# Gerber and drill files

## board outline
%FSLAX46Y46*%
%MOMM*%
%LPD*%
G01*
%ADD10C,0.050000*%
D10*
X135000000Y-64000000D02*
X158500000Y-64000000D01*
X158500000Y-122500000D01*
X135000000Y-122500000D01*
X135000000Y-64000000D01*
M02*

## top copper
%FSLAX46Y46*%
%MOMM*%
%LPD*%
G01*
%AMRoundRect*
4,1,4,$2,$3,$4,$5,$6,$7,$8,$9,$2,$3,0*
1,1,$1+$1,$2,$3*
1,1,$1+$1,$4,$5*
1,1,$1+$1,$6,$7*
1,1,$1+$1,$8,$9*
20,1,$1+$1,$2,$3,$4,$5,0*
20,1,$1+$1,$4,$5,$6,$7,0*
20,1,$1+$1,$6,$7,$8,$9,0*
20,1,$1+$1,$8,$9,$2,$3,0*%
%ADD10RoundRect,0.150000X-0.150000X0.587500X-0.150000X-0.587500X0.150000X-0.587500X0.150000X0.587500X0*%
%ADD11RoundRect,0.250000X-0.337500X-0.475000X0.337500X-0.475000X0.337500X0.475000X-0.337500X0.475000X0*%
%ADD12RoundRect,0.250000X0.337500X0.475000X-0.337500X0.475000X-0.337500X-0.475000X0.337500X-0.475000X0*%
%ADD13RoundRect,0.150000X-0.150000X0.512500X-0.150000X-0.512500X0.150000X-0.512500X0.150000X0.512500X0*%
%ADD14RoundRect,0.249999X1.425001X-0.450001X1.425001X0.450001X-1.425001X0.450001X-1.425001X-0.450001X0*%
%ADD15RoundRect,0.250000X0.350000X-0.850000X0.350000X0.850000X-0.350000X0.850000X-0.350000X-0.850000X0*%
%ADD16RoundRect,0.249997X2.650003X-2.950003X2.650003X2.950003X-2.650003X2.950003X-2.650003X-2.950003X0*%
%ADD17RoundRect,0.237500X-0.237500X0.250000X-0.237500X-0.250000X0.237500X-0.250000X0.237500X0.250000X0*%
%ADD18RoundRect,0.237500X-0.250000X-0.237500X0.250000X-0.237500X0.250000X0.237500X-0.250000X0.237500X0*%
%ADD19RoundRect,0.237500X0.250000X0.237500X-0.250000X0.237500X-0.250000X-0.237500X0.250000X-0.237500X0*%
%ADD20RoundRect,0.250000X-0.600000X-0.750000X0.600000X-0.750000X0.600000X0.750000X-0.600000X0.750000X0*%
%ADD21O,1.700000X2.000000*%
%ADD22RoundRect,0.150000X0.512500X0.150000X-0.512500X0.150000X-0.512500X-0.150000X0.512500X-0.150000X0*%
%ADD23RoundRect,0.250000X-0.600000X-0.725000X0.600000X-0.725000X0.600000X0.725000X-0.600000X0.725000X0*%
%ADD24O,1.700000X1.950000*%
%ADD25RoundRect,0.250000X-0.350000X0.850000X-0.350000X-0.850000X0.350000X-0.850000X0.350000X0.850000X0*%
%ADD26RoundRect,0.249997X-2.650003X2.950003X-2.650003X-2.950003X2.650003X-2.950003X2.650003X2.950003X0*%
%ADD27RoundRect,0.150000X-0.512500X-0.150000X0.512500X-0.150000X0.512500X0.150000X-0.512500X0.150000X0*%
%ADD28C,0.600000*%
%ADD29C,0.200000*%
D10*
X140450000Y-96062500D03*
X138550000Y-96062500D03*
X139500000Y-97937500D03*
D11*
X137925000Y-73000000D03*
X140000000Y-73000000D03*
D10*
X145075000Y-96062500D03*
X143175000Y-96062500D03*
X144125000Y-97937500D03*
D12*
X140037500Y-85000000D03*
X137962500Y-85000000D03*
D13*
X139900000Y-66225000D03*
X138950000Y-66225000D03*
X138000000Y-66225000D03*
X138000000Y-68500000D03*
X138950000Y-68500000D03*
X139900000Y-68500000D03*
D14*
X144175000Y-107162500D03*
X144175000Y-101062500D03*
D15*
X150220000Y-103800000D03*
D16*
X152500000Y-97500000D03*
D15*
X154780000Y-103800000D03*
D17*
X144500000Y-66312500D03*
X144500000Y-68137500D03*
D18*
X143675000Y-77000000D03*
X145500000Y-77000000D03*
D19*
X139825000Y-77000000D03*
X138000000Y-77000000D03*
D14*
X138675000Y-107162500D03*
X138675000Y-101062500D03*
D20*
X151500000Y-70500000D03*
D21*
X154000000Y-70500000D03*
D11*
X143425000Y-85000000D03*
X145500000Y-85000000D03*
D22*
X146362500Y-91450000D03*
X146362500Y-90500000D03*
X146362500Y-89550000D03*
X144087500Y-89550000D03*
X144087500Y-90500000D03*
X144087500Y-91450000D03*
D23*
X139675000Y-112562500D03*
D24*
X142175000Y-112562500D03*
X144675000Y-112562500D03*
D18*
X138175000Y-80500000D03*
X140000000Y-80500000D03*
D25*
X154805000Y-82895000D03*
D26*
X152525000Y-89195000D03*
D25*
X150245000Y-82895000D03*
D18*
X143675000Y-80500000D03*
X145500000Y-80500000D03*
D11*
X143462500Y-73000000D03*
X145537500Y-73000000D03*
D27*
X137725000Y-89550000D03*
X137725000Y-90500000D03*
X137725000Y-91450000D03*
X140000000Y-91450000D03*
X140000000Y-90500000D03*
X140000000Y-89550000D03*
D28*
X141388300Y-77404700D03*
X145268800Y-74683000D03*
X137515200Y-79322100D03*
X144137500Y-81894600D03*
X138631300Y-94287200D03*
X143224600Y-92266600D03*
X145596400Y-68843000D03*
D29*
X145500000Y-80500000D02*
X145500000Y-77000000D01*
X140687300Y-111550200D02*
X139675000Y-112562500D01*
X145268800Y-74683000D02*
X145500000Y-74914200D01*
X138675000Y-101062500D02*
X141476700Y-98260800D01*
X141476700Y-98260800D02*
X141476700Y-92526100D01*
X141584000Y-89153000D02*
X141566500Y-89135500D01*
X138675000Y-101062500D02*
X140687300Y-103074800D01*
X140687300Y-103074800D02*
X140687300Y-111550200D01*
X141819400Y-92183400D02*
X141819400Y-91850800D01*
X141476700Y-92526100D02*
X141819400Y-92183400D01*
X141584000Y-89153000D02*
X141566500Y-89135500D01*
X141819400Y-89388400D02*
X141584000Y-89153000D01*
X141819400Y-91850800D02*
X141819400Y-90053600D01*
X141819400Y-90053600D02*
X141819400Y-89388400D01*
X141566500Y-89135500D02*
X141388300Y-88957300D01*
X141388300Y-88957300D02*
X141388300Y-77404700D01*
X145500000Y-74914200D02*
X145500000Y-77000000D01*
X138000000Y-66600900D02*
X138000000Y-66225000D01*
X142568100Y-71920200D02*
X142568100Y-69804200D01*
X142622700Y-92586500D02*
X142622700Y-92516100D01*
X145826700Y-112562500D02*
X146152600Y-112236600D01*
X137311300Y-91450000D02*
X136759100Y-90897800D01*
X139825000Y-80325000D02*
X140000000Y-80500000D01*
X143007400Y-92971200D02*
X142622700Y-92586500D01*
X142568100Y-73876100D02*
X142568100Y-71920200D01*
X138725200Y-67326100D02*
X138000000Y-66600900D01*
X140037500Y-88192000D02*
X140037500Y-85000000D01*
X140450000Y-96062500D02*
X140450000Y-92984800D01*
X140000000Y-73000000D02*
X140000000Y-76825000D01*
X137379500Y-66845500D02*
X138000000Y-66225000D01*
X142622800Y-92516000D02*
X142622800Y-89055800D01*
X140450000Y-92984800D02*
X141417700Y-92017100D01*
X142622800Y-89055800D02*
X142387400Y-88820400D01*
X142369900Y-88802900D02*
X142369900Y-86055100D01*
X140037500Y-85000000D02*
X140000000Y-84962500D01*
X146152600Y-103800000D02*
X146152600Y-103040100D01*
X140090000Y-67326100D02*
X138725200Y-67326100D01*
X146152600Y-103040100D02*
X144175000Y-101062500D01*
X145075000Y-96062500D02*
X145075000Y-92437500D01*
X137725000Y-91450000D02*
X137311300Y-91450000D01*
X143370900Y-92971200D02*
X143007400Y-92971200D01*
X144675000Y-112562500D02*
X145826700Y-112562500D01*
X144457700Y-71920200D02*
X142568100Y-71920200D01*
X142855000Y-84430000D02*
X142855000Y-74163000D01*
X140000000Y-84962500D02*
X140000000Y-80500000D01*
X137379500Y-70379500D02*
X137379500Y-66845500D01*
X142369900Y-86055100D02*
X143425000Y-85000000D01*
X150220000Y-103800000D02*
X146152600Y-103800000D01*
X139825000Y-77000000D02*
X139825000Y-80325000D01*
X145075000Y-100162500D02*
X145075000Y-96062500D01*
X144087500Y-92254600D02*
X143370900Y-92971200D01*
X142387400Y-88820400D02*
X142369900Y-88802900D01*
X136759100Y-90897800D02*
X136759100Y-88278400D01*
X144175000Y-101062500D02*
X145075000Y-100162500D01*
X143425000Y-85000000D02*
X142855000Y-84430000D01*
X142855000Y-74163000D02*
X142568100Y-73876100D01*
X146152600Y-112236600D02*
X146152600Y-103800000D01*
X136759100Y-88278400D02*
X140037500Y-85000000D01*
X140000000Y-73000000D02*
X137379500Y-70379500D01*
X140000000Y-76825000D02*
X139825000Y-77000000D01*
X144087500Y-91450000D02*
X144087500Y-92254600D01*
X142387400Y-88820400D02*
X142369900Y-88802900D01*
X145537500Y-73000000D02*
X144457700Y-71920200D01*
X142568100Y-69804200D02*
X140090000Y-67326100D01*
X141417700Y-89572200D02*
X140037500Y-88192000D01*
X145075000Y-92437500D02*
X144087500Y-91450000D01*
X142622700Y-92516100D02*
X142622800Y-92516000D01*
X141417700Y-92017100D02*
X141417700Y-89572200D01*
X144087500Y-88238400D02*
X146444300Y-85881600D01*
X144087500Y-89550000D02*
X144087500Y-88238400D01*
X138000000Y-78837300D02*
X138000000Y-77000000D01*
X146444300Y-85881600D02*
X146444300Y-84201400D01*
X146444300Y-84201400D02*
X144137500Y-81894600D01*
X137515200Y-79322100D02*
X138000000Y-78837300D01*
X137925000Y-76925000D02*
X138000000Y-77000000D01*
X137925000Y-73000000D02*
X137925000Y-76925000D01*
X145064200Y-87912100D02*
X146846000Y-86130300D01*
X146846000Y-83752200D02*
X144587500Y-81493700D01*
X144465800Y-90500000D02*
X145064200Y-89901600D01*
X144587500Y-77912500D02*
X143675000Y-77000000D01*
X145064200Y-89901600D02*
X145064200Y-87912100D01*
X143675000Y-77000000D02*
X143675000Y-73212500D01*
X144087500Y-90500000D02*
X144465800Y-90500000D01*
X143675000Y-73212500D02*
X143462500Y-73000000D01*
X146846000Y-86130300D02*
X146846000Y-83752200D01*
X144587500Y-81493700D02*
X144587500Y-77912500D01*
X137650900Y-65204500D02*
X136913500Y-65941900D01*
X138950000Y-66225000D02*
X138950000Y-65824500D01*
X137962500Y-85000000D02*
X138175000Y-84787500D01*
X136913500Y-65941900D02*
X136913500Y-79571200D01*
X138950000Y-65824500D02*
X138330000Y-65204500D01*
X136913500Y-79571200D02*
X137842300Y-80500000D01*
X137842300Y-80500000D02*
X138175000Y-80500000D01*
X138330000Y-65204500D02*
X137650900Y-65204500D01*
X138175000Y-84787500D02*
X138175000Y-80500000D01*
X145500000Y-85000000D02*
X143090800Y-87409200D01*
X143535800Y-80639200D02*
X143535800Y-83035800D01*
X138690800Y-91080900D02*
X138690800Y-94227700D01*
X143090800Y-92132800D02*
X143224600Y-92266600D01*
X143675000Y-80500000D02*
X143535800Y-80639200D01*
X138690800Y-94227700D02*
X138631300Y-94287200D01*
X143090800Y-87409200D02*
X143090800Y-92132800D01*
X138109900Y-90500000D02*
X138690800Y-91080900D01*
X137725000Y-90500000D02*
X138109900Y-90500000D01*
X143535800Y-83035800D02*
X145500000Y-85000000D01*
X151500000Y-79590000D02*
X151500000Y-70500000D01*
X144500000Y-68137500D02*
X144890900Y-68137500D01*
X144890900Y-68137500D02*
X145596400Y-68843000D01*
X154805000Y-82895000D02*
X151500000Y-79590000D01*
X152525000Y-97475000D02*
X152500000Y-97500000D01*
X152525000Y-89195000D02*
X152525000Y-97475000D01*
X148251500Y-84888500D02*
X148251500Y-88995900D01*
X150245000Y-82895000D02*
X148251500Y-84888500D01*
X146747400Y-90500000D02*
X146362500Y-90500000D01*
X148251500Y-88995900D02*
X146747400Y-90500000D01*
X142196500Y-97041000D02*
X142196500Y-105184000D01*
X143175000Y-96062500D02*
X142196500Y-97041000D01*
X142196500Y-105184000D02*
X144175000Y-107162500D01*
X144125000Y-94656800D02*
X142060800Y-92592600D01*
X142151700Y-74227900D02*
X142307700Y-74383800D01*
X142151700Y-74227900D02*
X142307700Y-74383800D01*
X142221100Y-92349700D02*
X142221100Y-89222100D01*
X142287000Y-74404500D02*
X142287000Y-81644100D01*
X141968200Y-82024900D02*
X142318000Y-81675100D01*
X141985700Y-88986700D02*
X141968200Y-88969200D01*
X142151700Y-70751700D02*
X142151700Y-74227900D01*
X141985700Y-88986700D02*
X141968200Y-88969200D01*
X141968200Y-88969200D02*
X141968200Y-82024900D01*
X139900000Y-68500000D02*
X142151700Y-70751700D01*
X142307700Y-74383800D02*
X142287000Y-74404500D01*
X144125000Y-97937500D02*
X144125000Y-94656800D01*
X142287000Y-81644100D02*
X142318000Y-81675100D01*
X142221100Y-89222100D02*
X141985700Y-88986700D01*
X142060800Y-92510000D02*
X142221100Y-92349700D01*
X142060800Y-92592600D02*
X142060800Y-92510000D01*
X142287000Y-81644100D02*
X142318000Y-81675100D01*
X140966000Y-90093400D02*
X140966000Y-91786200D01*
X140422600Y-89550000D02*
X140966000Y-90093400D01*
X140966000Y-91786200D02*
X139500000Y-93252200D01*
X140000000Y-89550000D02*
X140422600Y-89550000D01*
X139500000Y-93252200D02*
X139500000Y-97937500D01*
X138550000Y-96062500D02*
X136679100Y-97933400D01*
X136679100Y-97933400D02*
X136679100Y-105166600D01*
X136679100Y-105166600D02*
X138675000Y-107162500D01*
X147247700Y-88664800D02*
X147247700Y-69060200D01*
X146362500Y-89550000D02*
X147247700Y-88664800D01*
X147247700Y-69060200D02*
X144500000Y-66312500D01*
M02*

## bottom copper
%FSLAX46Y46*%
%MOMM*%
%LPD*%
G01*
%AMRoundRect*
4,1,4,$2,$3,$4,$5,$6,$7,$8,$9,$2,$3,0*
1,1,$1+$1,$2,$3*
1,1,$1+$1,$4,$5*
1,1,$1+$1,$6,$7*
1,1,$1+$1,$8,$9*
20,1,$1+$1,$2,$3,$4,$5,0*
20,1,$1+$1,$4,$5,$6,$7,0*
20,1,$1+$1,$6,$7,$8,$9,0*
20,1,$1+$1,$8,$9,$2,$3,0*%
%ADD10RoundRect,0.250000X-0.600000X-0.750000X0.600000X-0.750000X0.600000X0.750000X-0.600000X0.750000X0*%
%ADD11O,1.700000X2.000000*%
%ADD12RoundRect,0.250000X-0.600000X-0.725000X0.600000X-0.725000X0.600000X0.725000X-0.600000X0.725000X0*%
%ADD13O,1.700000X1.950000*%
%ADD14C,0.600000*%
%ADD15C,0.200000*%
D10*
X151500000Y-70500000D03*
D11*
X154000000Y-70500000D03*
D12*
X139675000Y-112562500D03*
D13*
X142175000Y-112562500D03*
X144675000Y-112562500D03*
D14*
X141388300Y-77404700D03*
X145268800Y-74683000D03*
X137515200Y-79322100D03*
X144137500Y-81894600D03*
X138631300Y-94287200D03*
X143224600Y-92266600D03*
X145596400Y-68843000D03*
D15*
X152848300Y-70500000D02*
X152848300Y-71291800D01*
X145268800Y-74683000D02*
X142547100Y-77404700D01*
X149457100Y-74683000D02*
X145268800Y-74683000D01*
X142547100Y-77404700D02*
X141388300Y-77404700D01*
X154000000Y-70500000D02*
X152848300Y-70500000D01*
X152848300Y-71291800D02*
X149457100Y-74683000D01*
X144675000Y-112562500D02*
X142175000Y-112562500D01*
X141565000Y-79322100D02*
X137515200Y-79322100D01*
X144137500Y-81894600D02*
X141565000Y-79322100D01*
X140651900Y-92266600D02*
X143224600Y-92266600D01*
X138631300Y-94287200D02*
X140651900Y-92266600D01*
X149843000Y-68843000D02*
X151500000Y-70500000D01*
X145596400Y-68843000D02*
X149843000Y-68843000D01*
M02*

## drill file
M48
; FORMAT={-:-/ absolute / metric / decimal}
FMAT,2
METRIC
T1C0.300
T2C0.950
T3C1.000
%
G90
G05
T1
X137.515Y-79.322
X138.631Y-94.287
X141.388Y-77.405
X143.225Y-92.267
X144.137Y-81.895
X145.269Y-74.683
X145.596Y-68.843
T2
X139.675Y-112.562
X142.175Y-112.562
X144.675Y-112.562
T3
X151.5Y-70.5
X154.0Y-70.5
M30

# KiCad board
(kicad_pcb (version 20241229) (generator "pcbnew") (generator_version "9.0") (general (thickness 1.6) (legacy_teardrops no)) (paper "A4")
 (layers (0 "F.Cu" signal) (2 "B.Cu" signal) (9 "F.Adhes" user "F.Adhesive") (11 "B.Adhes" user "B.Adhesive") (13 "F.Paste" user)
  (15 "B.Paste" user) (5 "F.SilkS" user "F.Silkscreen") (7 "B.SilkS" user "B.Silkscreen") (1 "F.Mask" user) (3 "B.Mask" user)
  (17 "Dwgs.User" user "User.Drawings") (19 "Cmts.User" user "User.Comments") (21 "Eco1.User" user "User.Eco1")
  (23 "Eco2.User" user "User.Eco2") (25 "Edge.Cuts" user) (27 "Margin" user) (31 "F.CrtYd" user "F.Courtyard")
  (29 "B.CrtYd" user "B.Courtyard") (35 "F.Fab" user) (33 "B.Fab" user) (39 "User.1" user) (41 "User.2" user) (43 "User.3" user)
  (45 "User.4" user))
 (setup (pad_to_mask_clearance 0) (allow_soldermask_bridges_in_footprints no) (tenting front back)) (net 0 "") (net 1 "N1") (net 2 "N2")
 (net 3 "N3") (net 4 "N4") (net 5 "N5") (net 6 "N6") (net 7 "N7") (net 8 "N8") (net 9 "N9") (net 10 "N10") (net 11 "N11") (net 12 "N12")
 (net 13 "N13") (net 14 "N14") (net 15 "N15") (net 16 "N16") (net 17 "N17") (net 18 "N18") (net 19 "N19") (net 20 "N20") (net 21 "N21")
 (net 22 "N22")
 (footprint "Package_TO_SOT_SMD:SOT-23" (layer "F.Cu") (at 139.5 97 -90)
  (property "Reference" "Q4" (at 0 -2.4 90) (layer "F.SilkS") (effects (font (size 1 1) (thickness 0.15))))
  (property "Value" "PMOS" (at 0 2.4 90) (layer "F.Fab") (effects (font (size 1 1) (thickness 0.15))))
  (pad "1" smd roundrect (at -0.9375 -0.95 270) (size 1.475 0.6) (layers "F.Cu" "F.Mask" "F.Paste") (roundrect_rratio 0.25) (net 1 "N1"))
  (pad "2" smd roundrect (at -0.9375 0.95 270) (size 1.475 0.6) (layers "F.Cu" "F.Mask" "F.Paste") (roundrect_rratio 0.25) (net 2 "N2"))
  (pad "3" smd roundrect (at 0.9375 0 270) (size 1.475 0.6) (layers "F.Cu" "F.Mask" "F.Paste") (roundrect_rratio 0.25) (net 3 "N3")))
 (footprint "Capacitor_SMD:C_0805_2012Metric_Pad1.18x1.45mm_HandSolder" (layer "F.Cu") (at 138.9625 73)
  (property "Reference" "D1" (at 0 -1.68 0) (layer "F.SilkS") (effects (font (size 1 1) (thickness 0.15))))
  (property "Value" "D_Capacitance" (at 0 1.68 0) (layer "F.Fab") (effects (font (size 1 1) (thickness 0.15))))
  (pad "1" smd roundrect (at -1.0375 0) (size 1.175 1.45) (layers "F.Cu" "F.Mask" "F.Paste") (roundrect_rratio 0.212766) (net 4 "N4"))
  (pad "2" smd roundrect (at 1.0375 0) (size 1.175 1.45) (layers "F.Cu" "F.Mask" "F.Paste") (roundrect_rratio 0.212766) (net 1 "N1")))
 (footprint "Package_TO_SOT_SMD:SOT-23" (layer "F.Cu") (at 144.125 97 -90)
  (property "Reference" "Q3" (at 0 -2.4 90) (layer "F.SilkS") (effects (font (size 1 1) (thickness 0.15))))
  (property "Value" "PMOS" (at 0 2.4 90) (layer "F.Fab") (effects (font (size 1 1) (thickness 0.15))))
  (pad "1" smd roundrect (at -0.9375 -0.95 270) (size 1.475 0.6) (layers "F.Cu" "F.Mask" "F.Paste") (roundrect_rratio 0.25) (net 1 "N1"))
  (pad "2" smd roundrect (at -0.9375 0.95 270) (size 1.475 0.6) (layers "F.Cu" "F.Mask" "F.Paste") (roundrect_rratio 0.25) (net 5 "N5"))
  (pad "3" smd roundrect (at 0.9375 0 270) (size 1.475 0.6) (layers "F.Cu" "F.Mask" "F.Paste") (roundrect_rratio 0.25) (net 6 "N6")))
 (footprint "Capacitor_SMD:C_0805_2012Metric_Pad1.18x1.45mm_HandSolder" (layer "F.Cu") (at 139 85 180)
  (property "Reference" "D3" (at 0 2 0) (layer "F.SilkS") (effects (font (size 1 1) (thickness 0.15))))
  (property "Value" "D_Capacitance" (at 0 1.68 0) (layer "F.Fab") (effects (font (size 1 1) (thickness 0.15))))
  (pad "1" smd roundrect (at -1.0375 0 180) (size 1.175 1.45) (layers "F.Cu" "F.Mask" "F.Paste") (roundrect_rratio 0.212766) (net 1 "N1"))
  (pad "2" smd roundrect (at 1.0375 0 180) (size 1.175 1.45) (layers "F.Cu" "F.Mask" "F.Paste") (roundrect_rratio 0.212766) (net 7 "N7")))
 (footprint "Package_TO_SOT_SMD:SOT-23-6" (layer "F.Cu") (at 138.95 67.3625 -90)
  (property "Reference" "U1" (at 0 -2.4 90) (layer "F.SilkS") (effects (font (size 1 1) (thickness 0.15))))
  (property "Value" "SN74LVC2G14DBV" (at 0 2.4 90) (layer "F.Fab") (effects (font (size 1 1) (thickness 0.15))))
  (pad "1" smd roundrect (at -1.1375 -0.95 270) (size 1.325 0.6) (layers "F.Cu" "F.Mask" "F.Paste") (roundrect_rratio 0.25) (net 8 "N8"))
  (pad "2" smd roundrect (at -1.1375 0 270) (size 1.325 0.6) (layers "F.Cu" "F.Mask" "F.Paste") (roundrect_rratio 0.25) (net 7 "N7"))
  (pad "3" smd roundrect (at -1.1375 0.95 270) (size 1.325 0.6) (layers "F.Cu" "F.Mask" "F.Paste") (roundrect_rratio 0.25) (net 1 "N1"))
  (pad "4" smd roundrect (at 1.1375 0.95 270) (size 1.325 0.6) (layers "F.Cu" "F.Mask" "F.Paste") (roundrect_rratio 0.25) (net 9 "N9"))
  (pad "5" smd roundrect (at 1.1375 0 270) (size 1.325 0.6) (layers "F.Cu" "F.Mask" "F.Paste") (roundrect_rratio 0.25) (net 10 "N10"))
  (pad "6" smd roundrect (at 1.1375 -0.95 270) (size 1.325 0.6) (layers "F.Cu" "F.Mask" "F.Paste") (roundrect_rratio 0.25) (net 6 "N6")))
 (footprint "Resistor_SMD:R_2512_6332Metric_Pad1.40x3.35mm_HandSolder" (layer "F.Cu") (at 144.175 104.1125 90)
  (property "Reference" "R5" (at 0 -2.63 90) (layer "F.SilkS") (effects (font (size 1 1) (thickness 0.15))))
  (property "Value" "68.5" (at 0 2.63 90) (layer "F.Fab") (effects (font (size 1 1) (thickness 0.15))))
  (pad "1" smd roundrect (at -3.05 0 90) (size 1.4 3.35) (layers "F.Cu" "F.Mask" "F.Paste") (roundrect_rratio 0.178571) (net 5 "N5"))
  (pad "2" smd roundrect (at 3.05 0 90) (size 1.4 3.35) (layers "F.Cu" "F.Mask" "F.Paste") (roundrect_rratio 0.178571) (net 1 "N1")))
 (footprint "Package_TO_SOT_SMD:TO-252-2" (layer "F.Cu") (at 152.5 98.76 90)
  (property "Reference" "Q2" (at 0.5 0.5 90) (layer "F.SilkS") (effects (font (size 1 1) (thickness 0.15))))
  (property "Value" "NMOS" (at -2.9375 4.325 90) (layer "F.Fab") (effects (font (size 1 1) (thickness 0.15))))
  (pad "" smd roundrect (at -0.415 -1.525 90) (size 3.05 2.75) (layers "F.Paste") (roundrect_rratio 0.090909))
  (pad "" smd roundrect (at -0.415 1.525 90) (size 3.05 2.75) (layers "F.Paste") (roundrect_rratio 0.090909))
  (pad "" smd roundrect (at 2.935 -1.525 90) (size 3.05 2.75) (layers "F.Paste") (roundrect_rratio 0.090909))
  (pad "" smd roundrect (at 2.935 1.525 90) (size 3.05 2.75) (layers "F.Paste") (roundrect_rratio 0.090909))
  (pad "1" smd roundrect (at -5.04 -2.28 90) (size 2.2 1.2) (layers "F.Cu" "F.Mask" "F.Paste") (roundrect_rratio 0.208333) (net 1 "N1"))
  (pad "2" smd roundrect (at 1.26 0 90) (size 6.4 5.8) (layers "F.Cu" "F.Mask") (roundrect_rratio 0.043103) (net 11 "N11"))
  (pad "3" smd roundrect (at -5.04 2.28 90) (size 2.2 1.2) (layers "F.Cu" "F.Mask" "F.Paste") (roundrect_rratio 0.208333) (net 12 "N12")))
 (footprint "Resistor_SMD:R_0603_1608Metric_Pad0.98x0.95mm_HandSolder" (layer "F.Cu") (at 144.5 67.225 -90)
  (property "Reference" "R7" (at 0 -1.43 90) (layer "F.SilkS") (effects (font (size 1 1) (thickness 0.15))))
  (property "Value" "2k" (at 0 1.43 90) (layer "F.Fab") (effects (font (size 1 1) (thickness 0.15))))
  (pad "1" smd roundrect (at -0.9125 0 270) (size 0.975 0.95) (layers "F.Cu" "F.Mask" "F.Paste") (roundrect_rratio 0.25) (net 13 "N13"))
  (pad "2" smd roundrect (at 0.9125 0 270) (size 0.975 0.95) (layers "F.Cu" "F.Mask" "F.Paste") (roundrect_rratio 0.25) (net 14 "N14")))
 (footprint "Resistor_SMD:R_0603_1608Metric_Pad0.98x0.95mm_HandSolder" (layer "F.Cu") (at 144.5875 77)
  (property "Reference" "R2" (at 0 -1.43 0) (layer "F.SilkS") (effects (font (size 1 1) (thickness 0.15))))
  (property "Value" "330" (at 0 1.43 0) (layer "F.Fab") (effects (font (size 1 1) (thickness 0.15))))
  (pad "1" smd roundrect (at -0.9125 0) (size 0.975 0.95) (layers "F.Cu" "F.Mask" "F.Paste") (roundrect_rratio 0.25) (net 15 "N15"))
  (pad "2" smd roundrect (at 0.9125 0) (size 0.975 0.95) (layers "F.Cu" "F.Mask" "F.Paste") (roundrect_rratio 0.25) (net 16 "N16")))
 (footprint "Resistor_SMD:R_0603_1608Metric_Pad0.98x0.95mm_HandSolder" (layer "F.Cu") (at 138.9125 77 180)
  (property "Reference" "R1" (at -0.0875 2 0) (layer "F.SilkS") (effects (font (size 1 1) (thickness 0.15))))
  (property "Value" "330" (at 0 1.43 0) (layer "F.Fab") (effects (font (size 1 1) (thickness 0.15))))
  (pad "1" smd roundrect (at -0.9125 0 180) (size 0.975 0.95) (layers "F.Cu" "F.Mask" "F.Paste") (roundrect_rratio 0.25) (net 1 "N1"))
  (pad "2" smd roundrect (at 0.9125 0 180) (size 0.975 0.95) (layers "F.Cu" "F.Mask" "F.Paste") (roundrect_rratio 0.25) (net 4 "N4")))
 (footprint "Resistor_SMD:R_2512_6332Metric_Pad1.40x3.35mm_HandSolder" (layer "F.Cu") (at 138.675 104.1125 90)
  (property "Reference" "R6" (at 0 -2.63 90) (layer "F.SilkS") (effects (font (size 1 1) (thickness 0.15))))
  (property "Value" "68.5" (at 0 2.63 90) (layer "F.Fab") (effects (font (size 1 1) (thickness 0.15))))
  (pad "1" smd roundrect (at -3.05 0 90) (size 1.4 3.35) (layers "F.Cu" "F.Mask" "F.Paste") (roundrect_rratio 0.178571) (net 2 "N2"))
  (pad "2" smd roundrect (at 3.05 0 90) (size 1.4 3.35) (layers "F.Cu" "F.Mask" "F.Paste") (roundrect_rratio 0.178571) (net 16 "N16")))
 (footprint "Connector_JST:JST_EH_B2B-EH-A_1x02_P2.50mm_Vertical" (layer "F.Cu") (at 151.5 70.5)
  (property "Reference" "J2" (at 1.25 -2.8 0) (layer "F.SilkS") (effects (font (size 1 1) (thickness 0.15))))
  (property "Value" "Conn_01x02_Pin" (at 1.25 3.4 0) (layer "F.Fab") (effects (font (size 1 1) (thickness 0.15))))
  (pad "1" thru_hole roundrect (at 0 0) (size 1.7 2) (drill 1) (layers "*.Cu" "*.Mask") (remove_unused_layers no)
   (roundrect_rratio 0.147059) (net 14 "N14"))
  (pad "2" thru_hole oval (at 2.5 0) (size 1.7 2) (drill 1) (layers "*.Cu" "*.Mask") (remove_unused_layers no) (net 16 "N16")))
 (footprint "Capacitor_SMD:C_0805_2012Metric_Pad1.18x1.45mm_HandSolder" (layer "F.Cu") (at 144.4625 85)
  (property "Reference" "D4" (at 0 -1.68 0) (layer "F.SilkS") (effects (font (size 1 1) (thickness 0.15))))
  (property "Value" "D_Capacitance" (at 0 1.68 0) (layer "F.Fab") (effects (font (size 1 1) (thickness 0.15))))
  (pad "1" smd roundrect (at -1.0375 0) (size 1.175 1.45) (layers "F.Cu" "F.Mask" "F.Paste") (roundrect_rratio 0.212766) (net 1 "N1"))
  (pad "2" smd roundrect (at 1.0375 0) (size 1.175 1.45) (layers "F.Cu" "F.Mask" "F.Paste") (roundrect_rratio 0.212766) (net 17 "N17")))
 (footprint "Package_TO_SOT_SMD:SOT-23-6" (layer "F.Cu") (at 145.225 90.5 180)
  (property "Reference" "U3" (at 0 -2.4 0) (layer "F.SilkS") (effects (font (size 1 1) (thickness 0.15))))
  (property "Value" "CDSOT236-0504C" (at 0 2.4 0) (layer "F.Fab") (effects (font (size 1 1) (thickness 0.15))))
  (pad "1" smd roundrect (at -1.1375 -0.95 180) (size 1.325 0.6) (layers "F.Cu" "F.Mask" "F.Paste") (roundrect_rratio 0.25) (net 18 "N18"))
  (pad "2" smd roundrect (at -1.1375 0 180) (size 1.325 0.6) (layers "F.Cu" "F.Mask" "F.Paste") (roundrect_rratio 0.25) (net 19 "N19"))
  (pad "3" smd roundrect (at -1.1375 0.95 180) (size 1.325 0.6) (layers "F.Cu" "F.Mask" "F.Paste") (roundrect_rratio 0.25) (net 13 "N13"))
  (pad "4" smd roundrect (at 1.1375 0.95 180) (size 1.325 0.6) (layers "F.Cu" "F.Mask" "F.Paste") (roundrect_rratio 0.25) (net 4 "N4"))
  (pad "5" smd roundrect (at 1.1375 0 180) (size 1.325 0.6) (layers "F.Cu" "F.Mask" "F.Paste") (roundrect_rratio 0.25) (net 15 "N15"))
  (pad "6" smd roundrect (at 1.1375 -0.95 180) (size 1.325 0.6) (layers "F.Cu" "F.Mask" "F.Paste") (roundrect_rratio 0.25) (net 1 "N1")))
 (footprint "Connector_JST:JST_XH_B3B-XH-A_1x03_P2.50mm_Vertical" (layer "F.Cu") (at 139.675 112.5625)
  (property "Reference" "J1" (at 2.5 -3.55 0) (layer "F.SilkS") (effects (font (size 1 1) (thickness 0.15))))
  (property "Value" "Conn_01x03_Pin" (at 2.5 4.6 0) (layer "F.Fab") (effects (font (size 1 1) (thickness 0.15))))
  (pad "1" thru_hole roundrect (at 0 0) (size 1.7 1.95) (drill 0.95) (layers "*.Cu" "*.Mask") (remove_unused_layers no)
   (roundrect_rratio 0.147059) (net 16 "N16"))
  (pad "2" thru_hole oval (at 2.5 0) (size 1.7 1.95) (drill 0.95) (layers "*.Cu" "*.Mask") (remove_unused_layers no) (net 1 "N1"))
  (pad "3" thru_hole oval (at 5 0) (size 1.7 1.95) (drill 0.95) (layers "*.Cu" "*.Mask") (remove_unused_layers no) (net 1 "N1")))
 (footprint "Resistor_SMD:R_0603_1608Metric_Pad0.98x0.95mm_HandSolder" (layer "F.Cu") (at 139.0875 80.5)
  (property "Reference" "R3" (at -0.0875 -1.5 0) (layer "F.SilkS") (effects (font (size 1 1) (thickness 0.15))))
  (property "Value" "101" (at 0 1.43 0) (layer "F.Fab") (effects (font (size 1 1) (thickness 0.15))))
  (pad "1" smd roundrect (at -0.9125 0) (size 0.975 0.95) (layers "F.Cu" "F.Mask" "F.Paste") (roundrect_rratio 0.25) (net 7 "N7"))
  (pad "2" smd roundrect (at 0.9125 0) (size 0.975 0.95) (layers "F.Cu" "F.Mask" "F.Paste") (roundrect_rratio 0.25) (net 1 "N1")))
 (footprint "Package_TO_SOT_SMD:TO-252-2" (layer "F.Cu") (at 152.525 87.935 -90)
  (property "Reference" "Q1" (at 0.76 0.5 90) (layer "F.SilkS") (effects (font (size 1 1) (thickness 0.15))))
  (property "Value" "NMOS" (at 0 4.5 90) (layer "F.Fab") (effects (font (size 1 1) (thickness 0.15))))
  (pad "" smd roundrect (at -0.415 -1.525 270) (size 3.05 2.75) (layers "F.Paste") (roundrect_rratio 0.090909))
  (pad "" smd roundrect (at -0.415 1.525 270) (size 3.05 2.75) (layers "F.Paste") (roundrect_rratio 0.090909))
  (pad "" smd roundrect (at 2.935 -1.525 270) (size 3.05 2.75) (layers "F.Paste") (roundrect_rratio 0.090909))
  (pad "" smd roundrect (at 2.935 1.525 270) (size 3.05 2.75) (layers "F.Paste") (roundrect_rratio 0.090909))
  (pad "1" smd roundrect (at -5.04 -2.28 270) (size 2.2 1.2) (layers "F.Cu" "F.Mask" "F.Paste") (roundrect_rratio 0.208333) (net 14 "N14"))
  (pad "2" smd roundrect (at 1.26 0 270) (size 6.4 5.8) (layers "F.Cu" "F.Mask") (roundrect_rratio 0.043103) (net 11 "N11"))
  (pad "3" smd roundrect (at -5.04 2.28 270) (size 2.2 1.2) (layers "F.Cu" "F.Mask" "F.Paste") (roundrect_rratio 0.208333) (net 19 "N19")))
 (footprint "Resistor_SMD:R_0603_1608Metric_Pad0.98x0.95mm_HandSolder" (layer "F.Cu") (at 144.5875 80.5)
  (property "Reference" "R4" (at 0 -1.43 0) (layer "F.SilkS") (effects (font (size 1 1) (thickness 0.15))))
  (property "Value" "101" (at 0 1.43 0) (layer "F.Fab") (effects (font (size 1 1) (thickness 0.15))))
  (pad "1" smd roundrect (at -0.9125 0) (size 0.975 0.95) (layers "F.Cu" "F.Mask" "F.Paste") (roundrect_rratio 0.25) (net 17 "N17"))
  (pad "2" smd roundrect (at 0.9125 0) (size 0.975 0.95) (layers "F.Cu" "F.Mask" "F.Paste") (roundrect_rratio 0.25) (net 16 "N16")))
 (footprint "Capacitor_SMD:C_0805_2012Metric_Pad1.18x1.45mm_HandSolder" (layer "F.Cu") (at 144.5 73)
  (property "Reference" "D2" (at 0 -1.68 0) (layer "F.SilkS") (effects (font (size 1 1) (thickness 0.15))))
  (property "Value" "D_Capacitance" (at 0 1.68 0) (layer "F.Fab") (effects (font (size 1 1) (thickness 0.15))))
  (pad "1" smd roundrect (at -1.0375 0) (size 1.175 1.45) (layers "F.Cu" "F.Mask" "F.Paste") (roundrect_rratio 0.212766) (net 15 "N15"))
  (pad "2" smd roundrect (at 1.0375 0) (size 1.175 1.45) (layers "F.Cu" "F.Mask" "F.Paste") (roundrect_rratio 0.212766) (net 1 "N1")))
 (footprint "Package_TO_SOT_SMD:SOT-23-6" (layer "F.Cu") (at 138.8625 90.5)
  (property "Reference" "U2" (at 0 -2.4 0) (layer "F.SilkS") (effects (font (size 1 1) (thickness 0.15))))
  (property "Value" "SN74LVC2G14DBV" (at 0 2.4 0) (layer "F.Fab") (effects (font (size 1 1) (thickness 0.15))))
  (pad "1" smd roundrect (at -1.1375 -0.95) (size 1.325 0.6) (layers "F.Cu" "F.Mask" "F.Paste") (roundrect_rratio 0.25) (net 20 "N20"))
  (pad "2" smd roundrect (at -1.1375 0) (size 1.325 0.6) (layers "F.Cu" "F.Mask" "F.Paste") (roundrect_rratio 0.25) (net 17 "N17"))
  (pad "3" smd roundrect (at -1.1375 0.95) (size 1.325 0.6) (layers "F.Cu" "F.Mask" "F.Paste") (roundrect_rratio 0.25) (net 1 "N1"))
  (pad "4" smd roundrect (at 1.1375 0.95) (size 1.325 0.6) (layers "F.Cu" "F.Mask" "F.Paste") (roundrect_rratio 0.25) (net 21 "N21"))
  (pad "5" smd roundrect (at 1.1375 0) (size 1.325 0.6) (layers "F.Cu" "F.Mask" "F.Paste") (roundrect_rratio 0.25) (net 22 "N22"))
  (pad "6" smd roundrect (at 1.1375 -0.95) (size 1.325 0.6) (layers "F.Cu" "F.Mask" "F.Paste") (roundrect_rratio 0.25) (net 3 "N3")))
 (gr_rect (start 135 64) (end 158.5 122.5) (stroke (width 0.05) (type default)) (fill no) (layer "Edge.Cuts"))
 (segment (start 145.5 80.5) (end 145.5 77) (width 0.2) (layer "F.Cu") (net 16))
 (segment (start 140.6873 111.5502) (end 139.675 112.5625) (width 0.2) (layer "F.Cu") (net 16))
 (segment (start 145.2688 74.683) (end 145.5 74.9142) (width 0.2) (layer "F.Cu") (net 16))
 (segment (start 138.675 101.0625) (end 141.4767 98.2608) (width 0.2) (layer "F.Cu") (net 16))
 (segment (start 141.4767 98.2608) (end 141.4767 92.5261) (width 0.2) (layer "F.Cu") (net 16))
 (segment (start 141.584 89.153) (end 141.5665 89.1355) (width 0.2) (layer "F.Cu") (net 16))
 (segment (start 138.675 101.0625) (end 140.6873 103.0748) (width 0.2) (layer "F.Cu") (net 16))
 (segment (start 140.6873 103.0748) (end 140.6873 111.5502) (width 0.2) (layer "F.Cu") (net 16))
 (segment (start 141.8194 92.1834) (end 141.8194 91.8508) (width 0.2) (layer "F.Cu") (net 16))
 (segment (start 141.4767 92.5261) (end 141.8194 92.1834) (width 0.2) (layer "F.Cu") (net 16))
 (segment (start 141.584 89.153) (end 141.5665 89.1355) (width 0.2) (layer "F.Cu") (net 16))
 (segment (start 141.8194 89.3884) (end 141.584 89.153) (width 0.2) (layer "F.Cu") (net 16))
 (segment (start 141.8194 91.8508) (end 141.8194 90.0536) (width 0.2) (layer "F.Cu") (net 16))
 (segment (start 141.8194 90.0536) (end 141.8194 89.3884) (width 0.2) (layer "F.Cu") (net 16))
 (segment (start 141.5665 89.1355) (end 141.3883 88.9573) (width 0.2) (layer "F.Cu") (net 16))
 (segment (start 141.3883 88.9573) (end 141.3883 77.4047) (width 0.2) (layer "F.Cu") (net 16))
 (segment (start 145.5 74.9142) (end 145.5 77) (width 0.2) (layer "F.Cu") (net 16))
 (via (at 141.3883 77.4047) (size 0.6) (drill 0.3) (layers "F.Cu" "B.Cu") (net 16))
 (via (at 145.2688 74.683) (size 0.6) (drill 0.3) (layers "F.Cu" "B.Cu") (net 16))
 (segment (start 152.8483 70.5) (end 152.8483 71.2918) (width 0.2) (layer "B.Cu") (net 16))
 (segment (start 145.2688 74.683) (end 142.5471 77.4047) (width 0.2) (layer "B.Cu") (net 16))
 (segment (start 149.4571 74.683) (end 145.2688 74.683) (width 0.2) (layer "B.Cu") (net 16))
 (segment (start 142.5471 77.4047) (end 141.3883 77.4047) (width 0.2) (layer "B.Cu") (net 16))
 (segment (start 154 70.5) (end 152.8483 70.5) (width 0.2) (layer "B.Cu") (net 16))
 (segment (start 152.8483 71.2918) (end 149.4571 74.683) (width 0.2) (layer "B.Cu") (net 16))
 (segment (start 138 66.6009) (end 138 66.225) (width 0.2) (layer "F.Cu") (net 1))
 (segment (start 142.5681 71.9202) (end 142.5681 69.8042) (width 0.2) (layer "F.Cu") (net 1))
 (segment (start 142.6227 92.5865) (end 142.6227 92.5161) (width 0.2) (layer "F.Cu") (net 1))
 (segment (start 145.8267 112.5625) (end 146.1526 112.2366) (width 0.2) (layer "F.Cu") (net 1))
 (segment (start 137.3113 91.45) (end 136.7591 90.8978) (width 0.2) (layer "F.Cu") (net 1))
 (segment (start 139.825 80.325) (end 140 80.5) (width 0.2) (layer "F.Cu") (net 1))
 (segment (start 143.0074 92.9712) (end 142.6227 92.5865) (width 0.2) (layer "F.Cu") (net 1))
 (segment (start 142.5681 73.8761) (end 142.5681 71.9202) (width 0.2) (layer "F.Cu") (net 1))
 (segment (start 138.7252 67.3261) (end 138 66.6009) (width 0.2) (layer "F.Cu") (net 1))
 (segment (start 140.0375 88.192) (end 140.0375 85) (width 0.2) (layer "F.Cu") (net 1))
 (segment (start 140.45 96.0625) (end 140.45 92.9848) (width 0.2) (layer "F.Cu") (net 1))
 (segment (start 140 73) (end 140 76.825) (width 0.2) (layer "F.Cu") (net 1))
 (segment (start 137.3795 66.8455) (end 138 66.225) (width 0.2) (layer "F.Cu") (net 1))
 (segment (start 142.6228 92.516) (end 142.6228 89.0558) (width 0.2) (layer "F.Cu") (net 1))
 (segment (start 140.45 92.9848) (end 141.4177 92.0171) (width 0.2) (layer "F.Cu") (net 1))
 (segment (start 142.6228 89.0558) (end 142.3874 88.8204) (width 0.2) (layer "F.Cu") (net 1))
 (segment (start 142.3699 88.8029) (end 142.3699 86.0551) (width 0.2) (layer "F.Cu") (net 1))
 (segment (start 140.0375 85) (end 140 84.9625) (width 0.2) (layer "F.Cu") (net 1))
 (segment (start 146.1526 103.8) (end 146.1526 103.0401) (width 0.2) (layer "F.Cu") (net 1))
 (segment (start 140.09 67.3261) (end 138.7252 67.3261) (width 0.2) (layer "F.Cu") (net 1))
 (segment (start 146.1526 103.0401) (end 144.175 101.0625) (width 0.2) (layer "F.Cu") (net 1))
 (segment (start 145.075 96.0625) (end 145.075 92.4375) (width 0.2) (layer "F.Cu") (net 1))
 (segment (start 137.725 91.45) (end 137.3113 91.45) (width 0.2) (layer "F.Cu") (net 1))
 (segment (start 143.3709 92.9712) (end 143.0074 92.9712) (width 0.2) (layer "F.Cu") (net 1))
 (segment (start 144.675 112.5625) (end 145.8267 112.5625) (width 0.2) (layer "F.Cu") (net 1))
 (segment (start 144.4577 71.9202) (end 142.5681 71.9202) (width 0.2) (layer "F.Cu") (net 1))
 (segment (start 142.855 84.43) (end 142.855 74.163) (width 0.2) (layer "F.Cu") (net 1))
 (segment (start 140 84.9625) (end 140 80.5) (width 0.2) (layer "F.Cu") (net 1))
 (segment (start 137.3795 70.3795) (end 137.3795 66.8455) (width 0.2) (layer "F.Cu") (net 1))
 (segment (start 142.3699 86.0551) (end 143.425 85) (width 0.2) (layer "F.Cu") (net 1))
 (segment (start 150.22 103.8) (end 146.1526 103.8) (width 0.2) (layer "F.Cu") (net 1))
 (segment (start 139.825 77) (end 139.825 80.325) (width 0.2) (layer "F.Cu") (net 1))
 (segment (start 145.075 100.1625) (end 145.075 96.0625) (width 0.2) (layer "F.Cu") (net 1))
 (segment (start 144.0875 92.2546) (end 143.3709 92.9712) (width 0.2) (layer "F.Cu") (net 1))
 (segment (start 142.3874 88.8204) (end 142.3699 88.8029) (width 0.2) (layer "F.Cu") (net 1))
 (segment (start 136.7591 90.8978) (end 136.7591 88.2784) (width 0.2) (layer "F.Cu") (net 1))
 (segment (start 144.175 101.0625) (end 145.075 100.1625) (width 0.2) (layer "F.Cu") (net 1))
 (segment (start 143.425 85) (end 142.855 84.43) (width 0.2) (layer "F.Cu") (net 1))
 (segment (start 142.855 74.163) (end 142.5681 73.8761) (width 0.2) (layer "F.Cu") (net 1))
 (segment (start 146.1526 112.2366) (end 146.1526 103.8) (width 0.2) (layer "F.Cu") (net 1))
 (segment (start 136.7591 88.2784) (end 140.0375 85) (width 0.2) (layer "F.Cu") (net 1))
 (segment (start 140 73) (end 137.3795 70.3795) (width 0.2) (layer "F.Cu") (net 1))
 (segment (start 140 76.825) (end 139.825 77) (width 0.2) (layer "F.Cu") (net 1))
 (segment (start 144.0875 91.45) (end 144.0875 92.2546) (width 0.2) (layer "F.Cu") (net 1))
 (segment (start 142.3874 88.8204) (end 142.3699 88.8029) (width 0.2) (layer "F.Cu") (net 1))
 (segment (start 145.5375 73) (end 144.4577 71.9202) (width 0.2) (layer "F.Cu") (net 1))
 (segment (start 142.5681 69.8042) (end 140.09 67.3261) (width 0.2) (layer "F.Cu") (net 1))
 (segment (start 141.4177 89.5722) (end 140.0375 88.192) (width 0.2) (layer "F.Cu") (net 1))
 (segment (start 145.075 92.4375) (end 144.0875 91.45) (width 0.2) (layer "F.Cu") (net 1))
 (segment (start 142.6227 92.5161) (end 142.6228 92.516) (width 0.2) (layer "F.Cu") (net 1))
 (segment (start 141.4177 92.0171) (end 141.4177 89.5722) (width 0.2) (layer "F.Cu") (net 1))
 (segment (start 144.675 112.5625) (end 142.175 112.5625) (width 0.2) (layer "B.Cu") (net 1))
 (segment (start 144.0875 88.2384) (end 146.4443 85.8816) (width 0.2) (layer "F.Cu") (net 4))
 (segment (start 144.0875 89.55) (end 144.0875 88.2384) (width 0.2) (layer "F.Cu") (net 4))
 (segment (start 138 78.8373) (end 138 77) (width 0.2) (layer "F.Cu") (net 4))
 (segment (start 146.4443 85.8816) (end 146.4443 84.2014) (width 0.2) (layer "F.Cu") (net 4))
 (segment (start 146.4443 84.2014) (end 144.1375 81.8946) (width 0.2) (layer "F.Cu") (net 4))
 (segment (start 137.5152 79.3221) (end 138 78.8373) (width 0.2) (layer "F.Cu") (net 4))
 (segment (start 137.925 76.925) (end 138 77) (width 0.2) (layer "F.Cu") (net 4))
 (segment (start 137.925 73) (end 137.925 76.925) (width 0.2) (layer "F.Cu") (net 4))
 (via (at 137.5152 79.3221) (size 0.6) (drill 0.3) (layers "F.Cu" "B.Cu") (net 4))
 (via (at 144.1375 81.8946) (size 0.6) (drill 0.3) (layers "F.Cu" "B.Cu") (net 4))
 (segment (start 141.565 79.3221) (end 137.5152 79.3221) (width 0.2) (layer "B.Cu") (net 4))
 (segment (start 144.1375 81.8946) (end 141.565 79.3221) (width 0.2) (layer "B.Cu") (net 4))
 (segment (start 145.0642 87.9121) (end 146.846 86.1303) (width 0.2) (layer "F.Cu") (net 15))
 (segment (start 146.846 83.7522) (end 144.5875 81.4937) (width 0.2) (layer "F.Cu") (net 15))
 (segment (start 144.4658 90.5) (end 145.0642 89.9016) (width 0.2) (layer "F.Cu") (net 15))
 (segment (start 144.5875 77.9125) (end 143.675 77) (width 0.2) (layer "F.Cu") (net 15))
 (segment (start 145.0642 89.9016) (end 145.0642 87.9121) (width 0.2) (layer "F.Cu") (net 15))
 (segment (start 143.675 77) (end 143.675 73.2125) (width 0.2) (layer "F.Cu") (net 15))
 (segment (start 144.0875 90.5) (end 144.4658 90.5) (width 0.2) (layer "F.Cu") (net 15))
 (segment (start 143.675 73.2125) (end 143.4625 73) (width 0.2) (layer "F.Cu") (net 15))
 (segment (start 146.846 86.1303) (end 146.846 83.7522) (width 0.2) (layer "F.Cu") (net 15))
 (segment (start 144.5875 81.4937) (end 144.5875 77.9125) (width 0.2) (layer "F.Cu") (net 15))
 (segment (start 137.6509 65.2045) (end 136.9135 65.9419) (width 0.2) (layer "F.Cu") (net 7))
 (segment (start 138.95 66.225) (end 138.95 65.8245) (width 0.2) (layer "F.Cu") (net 7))
 (segment (start 137.9625 85) (end 138.175 84.7875) (width 0.2) (layer "F.Cu") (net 7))
 (segment (start 136.9135 65.9419) (end 136.9135 79.5712) (width 0.2) (layer "F.Cu") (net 7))
 (segment (start 138.95 65.8245) (end 138.33 65.2045) (width 0.2) (layer "F.Cu") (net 7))
 (segment (start 136.9135 79.5712) (end 137.8423 80.5) (width 0.2) (layer "F.Cu") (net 7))
 (segment (start 137.8423 80.5) (end 138.175 80.5) (width 0.2) (layer "F.Cu") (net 7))
 (segment (start 138.33 65.2045) (end 137.6509 65.2045) (width 0.2) (layer "F.Cu") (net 7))
 (segment (start 138.175 84.7875) (end 138.175 80.5) (width 0.2) (layer "F.Cu") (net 7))
 (segment (start 145.5 85) (end 143.0908 87.4092) (width 0.2) (layer "F.Cu") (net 17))
 (segment (start 143.5358 80.6392) (end 143.5358 83.0358) (width 0.2) (layer "F.Cu") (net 17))
 (segment (start 138.6908 91.0809) (end 138.6908 94.2277) (width 0.2) (layer "F.Cu") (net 17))
 (segment (start 143.0908 92.1328) (end 143.2246 92.2666) (width 0.2) (layer "F.Cu") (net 17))
 (segment (start 143.675 80.5) (end 143.5358 80.6392) (width 0.2) (layer "F.Cu") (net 17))
 (segment (start 138.6908 94.2277) (end 138.6313 94.2872) (width 0.2) (layer "F.Cu") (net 17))
 (segment (start 143.0908 87.4092) (end 143.0908 92.1328) (width 0.2) (layer "F.Cu") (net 17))
 (segment (start 138.1099 90.5) (end 138.6908 91.0809) (width 0.2) (layer "F.Cu") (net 17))
 (segment (start 137.725 90.5) (end 138.1099 90.5) (width 0.2) (layer "F.Cu") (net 17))
 (segment (start 143.5358 83.0358) (end 145.5 85) (width 0.2) (layer "F.Cu") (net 17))
 (via (at 138.6313 94.2872) (size 0.6) (drill 0.3) (layers "F.Cu" "B.Cu") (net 17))
 (via (at 143.2246 92.2666) (size 0.6) (drill 0.3) (layers "F.Cu" "B.Cu") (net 17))
 (segment (start 140.6519 92.2666) (end 143.2246 92.2666) (width 0.2) (layer "B.Cu") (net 17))
 (segment (start 138.6313 94.2872) (end 140.6519 92.2666) (width 0.2) (layer "B.Cu") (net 17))
 (segment (start 151.5 79.59) (end 151.5 70.5) (width 0.2) (layer "F.Cu") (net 14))
 (segment (start 144.5 68.1375) (end 144.8909 68.1375) (width 0.2) (layer "F.Cu") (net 14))
 (segment (start 144.8909 68.1375) (end 145.5964 68.843) (width 0.2) (layer "F.Cu") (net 14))
 (segment (start 154.805 82.895) (end 151.5 79.59) (width 0.2) (layer "F.Cu") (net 14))
 (via (at 145.5964 68.843) (size 0.6) (drill 0.3) (layers "F.Cu" "B.Cu") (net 14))
 (segment (start 149.843 68.843) (end 151.5 70.5) (width 0.2) (layer "B.Cu") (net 14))
 (segment (start 145.5964 68.843) (end 149.843 68.843) (width 0.2) (layer "B.Cu") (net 14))
 (segment (start 152.525 97.475) (end 152.5 97.5) (width 0.2) (layer "F.Cu") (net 11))
 (segment (start 152.525 89.195) (end 152.525 97.475) (width 0.2) (layer "F.Cu") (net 11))
 (segment (start 148.2515 84.8885) (end 148.2515 88.9959) (width 0.2) (layer "F.Cu") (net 19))
 (segment (start 150.245 82.895) (end 148.2515 84.8885) (width 0.2) (layer "F.Cu") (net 19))
 (segment (start 146.7474 90.5) (end 146.3625 90.5) (width 0.2) (layer "F.Cu") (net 19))
 (segment (start 148.2515 88.9959) (end 146.7474 90.5) (width 0.2) (layer "F.Cu") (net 19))
 (segment (start 142.1965 97.041) (end 142.1965 105.184) (width 0.2) (layer "F.Cu") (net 5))
 (segment (start 143.175 96.0625) (end 142.1965 97.041) (width 0.2) (layer "F.Cu") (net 5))
 (segment (start 142.1965 105.184) (end 144.175 107.1625) (width 0.2) (layer "F.Cu") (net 5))
 (segment (start 144.125 94.6568) (end 142.0608 92.5926) (width 0.2) (layer "F.Cu") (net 6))
 (segment (start 142.1517 74.2279) (end 142.3077 74.3838) (width 0.2) (layer "F.Cu") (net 6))
 (segment (start 142.1517 74.2279) (end 142.3077 74.3838) (width 0.2) (layer "F.Cu") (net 6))
 (segment (start 142.2211 92.3497) (end 142.2211 89.2221) (width 0.2) (layer "F.Cu") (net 6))
 (segment (start 142.287 74.4045) (end 142.287 81.6441) (width 0.2) (layer "F.Cu") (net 6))
 (segment (start 141.9682 82.0249) (end 142.318 81.6751) (width 0.2) (layer "F.Cu") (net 6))
 (segment (start 141.9857 88.9867) (end 141.9682 88.9692) (width 0.2) (layer "F.Cu") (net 6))
 (segment (start 142.1517 70.7517) (end 142.1517 74.2279) (width 0.2) (layer "F.Cu") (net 6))
 (segment (start 141.9857 88.9867) (end 141.9682 88.9692) (width 0.2) (layer "F.Cu") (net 6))
 (segment (start 141.9682 88.9692) (end 141.9682 82.0249) (width 0.2) (layer "F.Cu") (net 6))
 (segment (start 139.9 68.5) (end 142.1517 70.7517) (width 0.2) (layer "F.Cu") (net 6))
 (segment (start 142.3077 74.3838) (end 142.287 74.4045) (width 0.2) (layer "F.Cu") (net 6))
 (segment (start 144.125 97.9375) (end 144.125 94.6568) (width 0.2) (layer "F.Cu") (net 6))
 (segment (start 142.287 81.6441) (end 142.318 81.6751) (width 0.2) (layer "F.Cu") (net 6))
 (segment (start 142.2211 89.2221) (end 141.9857 88.9867) (width 0.2) (layer "F.Cu") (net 6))
 (segment (start 142.0608 92.51) (end 142.2211 92.3497) (width 0.2) (layer "F.Cu") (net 6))
 (segment (start 142.0608 92.5926) (end 142.0608 92.51) (width 0.2) (layer "F.Cu") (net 6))
 (segment (start 142.287 81.6441) (end 142.318 81.6751) (width 0.2) (layer "F.Cu") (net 6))
 (segment (start 140.966 90.0934) (end 140.966 91.7862) (width 0.2) (layer "F.Cu") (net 3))
 (segment (start 140.4226 89.55) (end 140.966 90.0934) (width 0.2) (layer "F.Cu") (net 3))
 (segment (start 140.966 91.7862) (end 139.5 93.2522) (width 0.2) (layer "F.Cu") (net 3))
 (segment (start 140 89.55) (end 140.4226 89.55) (width 0.2) (layer "F.Cu") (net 3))
 (segment (start 139.5 93.2522) (end 139.5 97.9375) (width 0.2) (layer "F.Cu") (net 3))
 (segment (start 138.55 96.0625) (end 136.6791 97.9334) (width 0.2) (layer "F.Cu") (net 2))
 (segment (start 136.6791 97.9334) (end 136.6791 105.1666) (width 0.2) (layer "F.Cu") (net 2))
 (segment (start 136.6791 105.1666) (end 138.675 107.1625) (width 0.2) (layer "F.Cu") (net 2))
 (segment (start 147.2477 88.6648) (end 147.2477 69.0602) (width 0.2) (layer "F.Cu") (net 13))
 (segment (start 146.3625 89.55) (end 147.2477 88.6648) (width 0.2) (layer "F.Cu") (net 13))
 (segment (start 147.2477 69.0602) (end 144.5 66.3125) (width 0.2) (layer "F.Cu") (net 13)))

